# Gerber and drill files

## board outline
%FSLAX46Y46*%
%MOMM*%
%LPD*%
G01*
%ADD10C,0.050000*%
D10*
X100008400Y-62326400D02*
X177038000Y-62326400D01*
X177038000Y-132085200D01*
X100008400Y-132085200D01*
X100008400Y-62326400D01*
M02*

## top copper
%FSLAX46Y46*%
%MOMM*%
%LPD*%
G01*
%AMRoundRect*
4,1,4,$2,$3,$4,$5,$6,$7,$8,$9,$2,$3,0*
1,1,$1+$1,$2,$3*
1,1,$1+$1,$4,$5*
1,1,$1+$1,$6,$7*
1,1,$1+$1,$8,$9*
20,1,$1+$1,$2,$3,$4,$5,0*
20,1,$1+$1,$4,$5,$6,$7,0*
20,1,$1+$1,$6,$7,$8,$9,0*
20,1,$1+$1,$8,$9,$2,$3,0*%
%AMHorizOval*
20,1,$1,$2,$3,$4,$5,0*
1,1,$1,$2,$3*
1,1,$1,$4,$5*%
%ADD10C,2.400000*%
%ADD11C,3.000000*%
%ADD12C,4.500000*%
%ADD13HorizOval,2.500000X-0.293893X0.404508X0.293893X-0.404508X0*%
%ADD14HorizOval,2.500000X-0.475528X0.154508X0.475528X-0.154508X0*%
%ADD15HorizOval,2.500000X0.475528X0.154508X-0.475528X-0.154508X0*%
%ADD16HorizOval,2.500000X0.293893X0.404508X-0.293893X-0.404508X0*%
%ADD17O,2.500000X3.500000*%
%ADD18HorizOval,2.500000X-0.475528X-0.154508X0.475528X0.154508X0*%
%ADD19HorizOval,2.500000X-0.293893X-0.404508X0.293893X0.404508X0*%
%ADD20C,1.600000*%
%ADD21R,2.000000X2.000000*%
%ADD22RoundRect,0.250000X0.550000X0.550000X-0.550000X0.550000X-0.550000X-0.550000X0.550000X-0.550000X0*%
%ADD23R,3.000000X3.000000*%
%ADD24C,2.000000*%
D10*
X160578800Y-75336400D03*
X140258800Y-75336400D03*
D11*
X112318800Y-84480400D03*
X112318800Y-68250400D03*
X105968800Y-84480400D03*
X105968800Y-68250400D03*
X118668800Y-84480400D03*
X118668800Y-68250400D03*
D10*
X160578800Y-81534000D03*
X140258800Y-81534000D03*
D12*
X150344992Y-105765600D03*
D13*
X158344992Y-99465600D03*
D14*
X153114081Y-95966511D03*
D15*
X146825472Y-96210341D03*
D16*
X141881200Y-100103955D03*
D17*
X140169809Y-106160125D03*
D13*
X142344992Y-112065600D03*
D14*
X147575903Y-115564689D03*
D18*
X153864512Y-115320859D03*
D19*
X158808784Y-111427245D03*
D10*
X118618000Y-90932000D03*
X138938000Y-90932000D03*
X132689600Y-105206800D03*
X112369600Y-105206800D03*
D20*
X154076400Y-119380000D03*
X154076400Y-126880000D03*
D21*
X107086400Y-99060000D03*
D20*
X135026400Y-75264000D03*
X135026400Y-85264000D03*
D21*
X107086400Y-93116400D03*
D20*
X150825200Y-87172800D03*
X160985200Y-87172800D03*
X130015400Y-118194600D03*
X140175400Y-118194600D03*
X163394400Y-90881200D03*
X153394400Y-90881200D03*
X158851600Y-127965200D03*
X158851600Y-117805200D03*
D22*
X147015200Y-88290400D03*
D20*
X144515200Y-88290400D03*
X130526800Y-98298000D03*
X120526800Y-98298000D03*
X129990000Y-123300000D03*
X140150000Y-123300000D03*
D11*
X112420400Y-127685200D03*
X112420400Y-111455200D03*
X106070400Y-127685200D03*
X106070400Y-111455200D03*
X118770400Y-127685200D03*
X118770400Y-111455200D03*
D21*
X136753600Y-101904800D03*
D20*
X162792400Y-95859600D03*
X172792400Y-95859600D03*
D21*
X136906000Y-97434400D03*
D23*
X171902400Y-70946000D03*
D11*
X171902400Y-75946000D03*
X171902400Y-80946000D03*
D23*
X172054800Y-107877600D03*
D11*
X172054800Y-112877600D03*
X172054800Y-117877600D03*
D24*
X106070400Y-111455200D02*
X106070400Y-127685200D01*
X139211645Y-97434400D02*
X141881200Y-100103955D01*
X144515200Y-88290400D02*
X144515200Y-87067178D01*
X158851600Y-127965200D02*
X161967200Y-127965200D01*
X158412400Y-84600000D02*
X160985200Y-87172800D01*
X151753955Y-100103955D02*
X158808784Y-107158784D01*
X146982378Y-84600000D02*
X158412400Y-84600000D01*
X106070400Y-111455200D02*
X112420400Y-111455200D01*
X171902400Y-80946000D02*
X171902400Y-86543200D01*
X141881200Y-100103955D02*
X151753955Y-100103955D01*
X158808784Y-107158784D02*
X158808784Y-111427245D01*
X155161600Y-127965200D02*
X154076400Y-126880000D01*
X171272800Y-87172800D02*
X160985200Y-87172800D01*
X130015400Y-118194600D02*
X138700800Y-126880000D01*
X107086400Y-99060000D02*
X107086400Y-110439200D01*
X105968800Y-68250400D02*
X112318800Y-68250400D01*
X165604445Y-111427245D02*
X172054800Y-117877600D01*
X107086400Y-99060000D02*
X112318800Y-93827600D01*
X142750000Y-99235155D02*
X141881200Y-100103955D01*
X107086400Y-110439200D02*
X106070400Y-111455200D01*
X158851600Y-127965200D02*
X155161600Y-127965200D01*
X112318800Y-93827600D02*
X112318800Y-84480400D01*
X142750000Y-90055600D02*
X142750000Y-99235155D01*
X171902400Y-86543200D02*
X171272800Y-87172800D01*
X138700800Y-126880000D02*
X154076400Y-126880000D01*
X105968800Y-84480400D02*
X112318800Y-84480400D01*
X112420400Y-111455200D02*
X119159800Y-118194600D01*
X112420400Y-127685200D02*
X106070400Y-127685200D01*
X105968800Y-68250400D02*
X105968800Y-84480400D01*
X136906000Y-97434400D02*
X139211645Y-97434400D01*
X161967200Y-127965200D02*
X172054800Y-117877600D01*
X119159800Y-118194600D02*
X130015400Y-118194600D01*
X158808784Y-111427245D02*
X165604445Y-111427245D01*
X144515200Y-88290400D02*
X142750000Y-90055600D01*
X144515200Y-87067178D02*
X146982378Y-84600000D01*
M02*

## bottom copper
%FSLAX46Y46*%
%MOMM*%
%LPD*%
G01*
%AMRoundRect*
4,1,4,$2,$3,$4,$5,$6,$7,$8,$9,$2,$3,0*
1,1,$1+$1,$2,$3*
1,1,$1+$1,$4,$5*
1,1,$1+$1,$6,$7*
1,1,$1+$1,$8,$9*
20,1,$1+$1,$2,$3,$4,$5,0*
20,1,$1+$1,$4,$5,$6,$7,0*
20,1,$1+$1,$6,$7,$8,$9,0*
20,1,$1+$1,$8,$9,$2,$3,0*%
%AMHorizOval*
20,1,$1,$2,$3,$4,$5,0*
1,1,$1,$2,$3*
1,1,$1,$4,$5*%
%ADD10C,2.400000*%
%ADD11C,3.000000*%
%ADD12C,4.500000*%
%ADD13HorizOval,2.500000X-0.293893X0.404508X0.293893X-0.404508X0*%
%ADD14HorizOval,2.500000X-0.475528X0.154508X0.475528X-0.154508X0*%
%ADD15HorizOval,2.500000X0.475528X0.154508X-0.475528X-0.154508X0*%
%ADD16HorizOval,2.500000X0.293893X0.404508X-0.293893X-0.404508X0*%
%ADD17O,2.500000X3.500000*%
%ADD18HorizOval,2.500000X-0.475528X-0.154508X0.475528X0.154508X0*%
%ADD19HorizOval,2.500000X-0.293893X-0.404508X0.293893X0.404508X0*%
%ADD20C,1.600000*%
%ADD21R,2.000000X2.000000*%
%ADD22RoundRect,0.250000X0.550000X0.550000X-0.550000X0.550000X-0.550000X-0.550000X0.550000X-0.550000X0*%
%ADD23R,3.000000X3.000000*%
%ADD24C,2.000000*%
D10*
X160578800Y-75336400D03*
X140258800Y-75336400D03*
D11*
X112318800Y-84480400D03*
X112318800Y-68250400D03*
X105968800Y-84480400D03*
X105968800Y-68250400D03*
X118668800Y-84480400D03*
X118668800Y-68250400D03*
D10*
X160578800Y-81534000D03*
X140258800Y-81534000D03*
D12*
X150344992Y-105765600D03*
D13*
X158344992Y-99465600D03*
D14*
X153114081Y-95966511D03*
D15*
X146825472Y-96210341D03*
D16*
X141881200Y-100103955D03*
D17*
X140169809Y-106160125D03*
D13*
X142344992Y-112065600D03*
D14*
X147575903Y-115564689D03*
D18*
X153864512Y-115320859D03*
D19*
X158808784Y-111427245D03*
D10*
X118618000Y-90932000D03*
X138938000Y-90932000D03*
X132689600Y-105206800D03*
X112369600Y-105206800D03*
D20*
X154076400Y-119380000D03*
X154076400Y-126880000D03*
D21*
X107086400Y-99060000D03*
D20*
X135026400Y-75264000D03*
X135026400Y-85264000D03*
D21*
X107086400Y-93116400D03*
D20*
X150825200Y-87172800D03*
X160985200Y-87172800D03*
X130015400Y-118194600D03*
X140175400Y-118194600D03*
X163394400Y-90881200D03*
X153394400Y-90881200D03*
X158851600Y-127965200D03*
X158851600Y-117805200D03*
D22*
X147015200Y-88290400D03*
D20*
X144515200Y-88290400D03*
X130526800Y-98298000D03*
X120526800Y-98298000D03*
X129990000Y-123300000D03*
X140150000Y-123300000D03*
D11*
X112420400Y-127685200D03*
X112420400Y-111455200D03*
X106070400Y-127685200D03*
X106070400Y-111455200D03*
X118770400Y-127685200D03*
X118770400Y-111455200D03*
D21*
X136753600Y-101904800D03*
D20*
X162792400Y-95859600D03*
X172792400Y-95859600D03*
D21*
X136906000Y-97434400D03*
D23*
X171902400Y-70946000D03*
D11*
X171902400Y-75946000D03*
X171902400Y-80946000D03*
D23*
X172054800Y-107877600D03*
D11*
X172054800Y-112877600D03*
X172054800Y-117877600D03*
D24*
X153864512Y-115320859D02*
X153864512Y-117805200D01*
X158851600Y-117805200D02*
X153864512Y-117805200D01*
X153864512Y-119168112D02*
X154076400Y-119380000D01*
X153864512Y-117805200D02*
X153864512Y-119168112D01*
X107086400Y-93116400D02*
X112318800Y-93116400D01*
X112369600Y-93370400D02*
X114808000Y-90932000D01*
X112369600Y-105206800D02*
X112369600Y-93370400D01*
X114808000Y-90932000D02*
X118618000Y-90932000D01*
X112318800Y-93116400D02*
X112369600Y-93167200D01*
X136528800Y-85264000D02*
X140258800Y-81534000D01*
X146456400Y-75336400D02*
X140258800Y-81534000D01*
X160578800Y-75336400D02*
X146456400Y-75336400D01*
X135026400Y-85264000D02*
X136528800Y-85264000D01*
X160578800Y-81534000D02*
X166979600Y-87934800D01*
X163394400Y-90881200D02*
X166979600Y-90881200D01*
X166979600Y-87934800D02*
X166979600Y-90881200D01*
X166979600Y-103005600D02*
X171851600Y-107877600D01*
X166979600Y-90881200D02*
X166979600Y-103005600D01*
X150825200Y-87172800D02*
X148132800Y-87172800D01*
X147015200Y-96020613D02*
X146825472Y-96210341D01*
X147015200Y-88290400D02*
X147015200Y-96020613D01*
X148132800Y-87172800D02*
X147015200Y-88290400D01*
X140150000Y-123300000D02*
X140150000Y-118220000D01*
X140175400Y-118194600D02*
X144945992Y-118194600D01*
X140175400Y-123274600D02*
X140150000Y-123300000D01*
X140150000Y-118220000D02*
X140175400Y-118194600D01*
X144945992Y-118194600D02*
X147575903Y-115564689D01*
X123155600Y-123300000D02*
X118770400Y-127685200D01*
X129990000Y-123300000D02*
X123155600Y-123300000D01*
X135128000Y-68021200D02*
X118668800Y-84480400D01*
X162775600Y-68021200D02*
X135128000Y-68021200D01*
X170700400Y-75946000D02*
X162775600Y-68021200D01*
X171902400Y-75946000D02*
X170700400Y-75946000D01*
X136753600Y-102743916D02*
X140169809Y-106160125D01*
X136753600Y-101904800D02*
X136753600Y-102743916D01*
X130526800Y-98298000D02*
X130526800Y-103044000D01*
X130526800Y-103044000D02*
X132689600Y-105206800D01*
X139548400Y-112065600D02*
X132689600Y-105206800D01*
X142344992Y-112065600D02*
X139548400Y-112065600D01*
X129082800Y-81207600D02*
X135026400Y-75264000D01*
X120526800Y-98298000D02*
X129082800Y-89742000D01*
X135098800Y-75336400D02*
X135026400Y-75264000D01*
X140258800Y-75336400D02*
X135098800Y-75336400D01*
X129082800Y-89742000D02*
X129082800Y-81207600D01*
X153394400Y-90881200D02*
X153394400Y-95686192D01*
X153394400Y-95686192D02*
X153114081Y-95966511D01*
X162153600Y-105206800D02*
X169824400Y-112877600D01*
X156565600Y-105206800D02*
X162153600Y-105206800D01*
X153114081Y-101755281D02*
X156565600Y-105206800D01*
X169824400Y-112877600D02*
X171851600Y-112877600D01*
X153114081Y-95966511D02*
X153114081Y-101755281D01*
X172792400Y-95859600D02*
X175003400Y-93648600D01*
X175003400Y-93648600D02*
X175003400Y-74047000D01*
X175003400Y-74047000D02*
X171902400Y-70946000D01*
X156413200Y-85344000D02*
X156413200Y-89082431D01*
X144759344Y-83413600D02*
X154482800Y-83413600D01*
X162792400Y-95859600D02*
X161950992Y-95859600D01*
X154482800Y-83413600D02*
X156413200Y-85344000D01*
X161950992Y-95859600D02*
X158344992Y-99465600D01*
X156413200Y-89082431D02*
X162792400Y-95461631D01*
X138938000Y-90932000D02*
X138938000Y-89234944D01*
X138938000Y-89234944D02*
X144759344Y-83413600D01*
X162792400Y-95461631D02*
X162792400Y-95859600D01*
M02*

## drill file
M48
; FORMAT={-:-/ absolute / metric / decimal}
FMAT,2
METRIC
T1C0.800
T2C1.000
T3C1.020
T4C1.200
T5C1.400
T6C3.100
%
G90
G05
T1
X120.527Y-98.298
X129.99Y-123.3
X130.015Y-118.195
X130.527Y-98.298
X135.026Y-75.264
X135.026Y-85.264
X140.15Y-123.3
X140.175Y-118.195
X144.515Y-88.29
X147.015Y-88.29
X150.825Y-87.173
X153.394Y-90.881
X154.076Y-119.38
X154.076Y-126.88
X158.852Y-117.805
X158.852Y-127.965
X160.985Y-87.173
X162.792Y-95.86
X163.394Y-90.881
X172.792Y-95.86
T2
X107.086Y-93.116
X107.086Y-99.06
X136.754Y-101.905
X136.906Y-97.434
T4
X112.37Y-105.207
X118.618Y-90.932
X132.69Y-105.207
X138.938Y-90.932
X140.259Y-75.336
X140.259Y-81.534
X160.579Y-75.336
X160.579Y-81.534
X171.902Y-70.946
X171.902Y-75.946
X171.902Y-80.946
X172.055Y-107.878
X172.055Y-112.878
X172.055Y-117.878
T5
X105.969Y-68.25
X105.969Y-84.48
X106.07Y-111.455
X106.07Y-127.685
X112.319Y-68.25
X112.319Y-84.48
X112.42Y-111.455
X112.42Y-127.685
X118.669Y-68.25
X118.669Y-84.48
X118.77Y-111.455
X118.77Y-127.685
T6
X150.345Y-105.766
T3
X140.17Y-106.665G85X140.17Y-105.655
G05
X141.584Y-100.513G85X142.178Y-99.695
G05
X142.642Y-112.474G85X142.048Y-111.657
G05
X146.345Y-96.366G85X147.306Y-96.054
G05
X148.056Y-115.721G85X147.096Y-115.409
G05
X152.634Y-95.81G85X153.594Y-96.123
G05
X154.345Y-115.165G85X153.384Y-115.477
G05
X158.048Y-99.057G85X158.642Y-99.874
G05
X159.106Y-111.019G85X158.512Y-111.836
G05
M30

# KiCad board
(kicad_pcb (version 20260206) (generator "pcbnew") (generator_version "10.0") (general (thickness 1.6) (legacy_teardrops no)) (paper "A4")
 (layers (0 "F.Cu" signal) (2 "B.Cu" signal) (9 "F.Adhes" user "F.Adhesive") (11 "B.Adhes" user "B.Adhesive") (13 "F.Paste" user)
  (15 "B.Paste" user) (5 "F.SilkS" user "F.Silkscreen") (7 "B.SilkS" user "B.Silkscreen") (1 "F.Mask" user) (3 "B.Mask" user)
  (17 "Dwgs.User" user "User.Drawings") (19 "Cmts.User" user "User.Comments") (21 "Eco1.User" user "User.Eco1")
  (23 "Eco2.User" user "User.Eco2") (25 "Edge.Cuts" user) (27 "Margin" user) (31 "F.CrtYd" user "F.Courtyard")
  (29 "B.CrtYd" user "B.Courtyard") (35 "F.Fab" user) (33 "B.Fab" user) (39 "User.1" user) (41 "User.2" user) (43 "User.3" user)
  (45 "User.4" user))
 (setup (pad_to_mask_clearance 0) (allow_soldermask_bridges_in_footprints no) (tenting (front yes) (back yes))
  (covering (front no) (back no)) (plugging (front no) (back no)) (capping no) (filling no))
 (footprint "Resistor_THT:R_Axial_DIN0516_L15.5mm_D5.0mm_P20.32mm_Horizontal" (layer "F.Cu") (at 160.5788 75.3364 180)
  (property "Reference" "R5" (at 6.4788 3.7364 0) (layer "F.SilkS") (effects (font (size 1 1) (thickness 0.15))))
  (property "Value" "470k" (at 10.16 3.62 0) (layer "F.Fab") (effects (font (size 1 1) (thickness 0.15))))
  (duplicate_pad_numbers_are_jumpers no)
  (pad "1" thru_hole circle (at 0 0 180) (size 2.4 2.4) (drill 1.2) (layers "*.Cu" "*.Mask") (remove_unused_layers no) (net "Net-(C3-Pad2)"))
  (pad "2" thru_hole circle (at 20.32 0 180) (size 2.4 2.4) (drill 1.2) (layers "*.Cu" "*.Mask") (remove_unused_layers no)
   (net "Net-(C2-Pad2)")))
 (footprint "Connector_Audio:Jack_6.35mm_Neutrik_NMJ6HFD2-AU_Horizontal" (layer "F.Cu") (at 118.6688 84.4804 180)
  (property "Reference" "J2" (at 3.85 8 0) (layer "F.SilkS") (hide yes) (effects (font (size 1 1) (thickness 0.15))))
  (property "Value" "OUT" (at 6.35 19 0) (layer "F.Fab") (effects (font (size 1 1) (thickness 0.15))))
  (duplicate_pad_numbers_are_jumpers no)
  (pad "R" thru_hole circle (at 6.35 0 180) (size 3 3) (drill 1.4) (layers "*.Cu" "*.Mask") (remove_unused_layers no) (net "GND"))
  (pad "RN" thru_hole circle (at 6.35 16.23 180) (size 3 3) (drill 1.4) (layers "*.Cu" "*.Mask") (remove_unused_layers no) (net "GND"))
  (pad "S" thru_hole circle (at 12.7 0 180) (size 3 3) (drill 1.4) (layers "*.Cu" "*.Mask") (remove_unused_layers no) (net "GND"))
  (pad "SN" thru_hole circle (at 12.7 16.23 180) (size 3 3) (drill 1.4) (layers "*.Cu" "*.Mask") (remove_unused_layers no) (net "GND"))
  (pad "T" thru_hole circle (at 0 0 180) (size 3 3) (drill 1.4) (layers "*.Cu" "*.Mask") (remove_unused_layers no) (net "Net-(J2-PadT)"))
  (pad "TN" thru_hole circle (at 0 16.23 180) (size 3 3) (drill 1.4) (layers "*.Cu" "*.Mask") (remove_unused_layers no)
   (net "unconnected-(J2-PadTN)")))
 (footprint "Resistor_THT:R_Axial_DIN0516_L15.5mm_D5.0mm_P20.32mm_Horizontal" (layer "F.Cu") (at 160.5788 81.534 180)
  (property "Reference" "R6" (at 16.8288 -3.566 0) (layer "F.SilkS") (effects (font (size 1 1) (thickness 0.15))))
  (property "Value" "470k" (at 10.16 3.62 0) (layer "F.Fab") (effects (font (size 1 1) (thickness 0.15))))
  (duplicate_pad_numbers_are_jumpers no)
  (pad "1" thru_hole circle (at 0 0 180) (size 2.4 2.4) (drill 1.2) (layers "*.Cu" "*.Mask") (remove_unused_layers no) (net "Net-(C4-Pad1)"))
  (pad "2" thru_hole circle (at 20.32 0 180) (size 2.4 2.4) (drill 1.2) (layers "*.Cu" "*.Mask") (remove_unused_layers no)
   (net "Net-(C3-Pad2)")))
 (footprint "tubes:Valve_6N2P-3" (layer "F.Cu") (at 158.344992 99.4656 90)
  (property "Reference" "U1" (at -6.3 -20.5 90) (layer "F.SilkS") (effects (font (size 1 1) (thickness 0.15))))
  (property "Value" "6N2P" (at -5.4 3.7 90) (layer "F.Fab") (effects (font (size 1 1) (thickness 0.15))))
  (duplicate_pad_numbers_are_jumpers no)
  (pad "" np_thru_hole circle (at -6.3 -8 90) (size 4.5 4.5) (drill 3.1) (layers "*.Cu" "*.Mask"))
  (pad "1" thru_hole oval (at 0 0 36) (size 2.5 3.5) (drill oval 1.02 2.03) (layers "*.Cu" "*.Mask") (remove_unused_layers no)
   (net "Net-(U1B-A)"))
  (pad "2" thru_hole oval (at 3.499089 -5.230911 72) (size 2.5 3.5) (drill oval 1.02 2.03) (layers "*.Cu" "*.Mask")
   (remove_unused_layers no) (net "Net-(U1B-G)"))
  (pad "3" thru_hole oval (at 3.255259 -11.51952 108) (size 2.5 3.5) (drill oval 1.02 2.03) (layers "*.Cu" "*.Mask")
   (remove_unused_layers no) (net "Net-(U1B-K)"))
  (pad "4" thru_hole oval (at -0.638355 -16.463792 144) (size 2.5 3.5) (drill oval 1.02 2.03) (layers "*.Cu" "*.Mask")
   (remove_unused_layers no) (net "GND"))
  (pad "5" thru_hole oval (at -6.694525 -18.175183 180) (size 2.5 3.5) (drill oval 1.02 2.03) (layers "*.Cu" "*.Mask")
   (remove_unused_layers no) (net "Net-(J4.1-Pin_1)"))
  (pad "6" thru_hole oval (at -12.6 -16 216) (size 2.5 3.5) (drill oval 1.02 2.03) (layers "*.Cu" "*.Mask") (remove_unused_layers no)
   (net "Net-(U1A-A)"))
  (pad "7" thru_hole oval (at -16.099089 -10.769089 252) (size 2.5 3.5) (drill oval 1.02 2.03) (layers "*.Cu" "*.Mask")
   (remove_unused_layers no) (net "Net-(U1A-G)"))
  (pad "8" thru_hole oval (at -15.855259 -4.48048 288) (size 2.5 3.5) (drill oval 1.02 2.03) (layers "*.Cu" "*.Mask")
   (remove_unused_layers no) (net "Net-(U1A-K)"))
  (pad "9" thru_hole oval (at -11.961645 0.463792 324) (size 2.5 3.5) (drill oval 1.02 2.03) (layers "*.Cu" "*.Mask")
   (remove_unused_layers no) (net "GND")))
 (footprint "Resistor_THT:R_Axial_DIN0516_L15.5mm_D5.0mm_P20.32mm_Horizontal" (layer "F.Cu") (at 118.618 90.932)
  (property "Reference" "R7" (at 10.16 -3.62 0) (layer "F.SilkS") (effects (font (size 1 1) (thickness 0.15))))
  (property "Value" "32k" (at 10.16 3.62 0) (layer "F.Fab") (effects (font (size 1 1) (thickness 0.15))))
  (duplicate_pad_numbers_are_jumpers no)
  (pad "1" thru_hole circle (at 0 0) (size 2.4 2.4) (drill 1.2) (layers "*.Cu" "*.Mask") (remove_unused_layers no) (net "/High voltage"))
  (pad "2" thru_hole circle (at 20.32 0) (size 2.4 2.4) (drill 1.2) (layers "*.Cu" "*.Mask") (remove_unused_layers no) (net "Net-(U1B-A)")))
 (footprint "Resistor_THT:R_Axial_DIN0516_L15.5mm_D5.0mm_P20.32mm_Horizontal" (layer "F.Cu") (at 132.6896 105.2068 180)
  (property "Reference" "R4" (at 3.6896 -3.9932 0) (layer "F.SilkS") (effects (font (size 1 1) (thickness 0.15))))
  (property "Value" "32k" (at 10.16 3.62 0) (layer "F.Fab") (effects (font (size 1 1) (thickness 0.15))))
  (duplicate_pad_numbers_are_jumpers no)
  (pad "1" thru_hole circle (at 0 0 180) (size 2.4 2.4) (drill 1.2) (layers "*.Cu" "*.Mask") (remove_unused_layers no) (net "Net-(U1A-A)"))
  (pad "2" thru_hole circle (at 20.32 0 180) (size 2.4 2.4) (drill 1.2) (layers "*.Cu" "*.Mask") (remove_unused_layers no)
   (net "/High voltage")))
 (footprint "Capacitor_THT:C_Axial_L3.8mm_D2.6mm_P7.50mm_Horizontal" (layer "F.Cu") (at 154.0764 119.38 -90)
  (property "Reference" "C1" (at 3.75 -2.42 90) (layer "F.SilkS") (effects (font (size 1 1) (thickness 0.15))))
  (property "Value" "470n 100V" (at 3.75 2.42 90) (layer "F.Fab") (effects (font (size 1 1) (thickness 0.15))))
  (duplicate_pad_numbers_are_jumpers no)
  (pad "1" thru_hole circle (at 0 0 270) (size 1.6 1.6) (drill 0.8) (layers "*.Cu" "*.Mask") (remove_unused_layers no) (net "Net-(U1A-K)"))
  (pad "2" thru_hole circle (at 7.5 0 270) (size 1.6 1.6) (drill 0.8) (layers "*.Cu" "*.Mask") (remove_unused_layers no) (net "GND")))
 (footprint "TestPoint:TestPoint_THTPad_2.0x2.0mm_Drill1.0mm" (layer "F.Cu") (at 107.0864 99.06)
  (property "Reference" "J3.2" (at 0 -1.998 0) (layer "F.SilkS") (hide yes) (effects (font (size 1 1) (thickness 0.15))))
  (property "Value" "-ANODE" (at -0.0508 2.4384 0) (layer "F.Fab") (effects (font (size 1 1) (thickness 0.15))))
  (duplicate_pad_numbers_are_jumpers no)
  (pad "1" thru_hole rect (at 0 0) (size 2 2) (drill 1) (layers "*.Cu" "*.Mask") (remove_unused_layers no) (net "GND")))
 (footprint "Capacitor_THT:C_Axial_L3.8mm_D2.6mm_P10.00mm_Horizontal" (layer "F.Cu") (at 135.0264 75.264 -90)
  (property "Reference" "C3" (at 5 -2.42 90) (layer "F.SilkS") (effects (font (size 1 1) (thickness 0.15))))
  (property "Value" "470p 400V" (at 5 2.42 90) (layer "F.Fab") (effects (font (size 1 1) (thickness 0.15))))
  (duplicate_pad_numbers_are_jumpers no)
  (pad "1" thru_hole circle (at 0 0 270) (size 1.6 1.6) (drill 0.8) (layers "*.Cu" "*.Mask") (remove_unused_layers no) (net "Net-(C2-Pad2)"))
  (pad "2" thru_hole circle (at 10 0 270) (size 1.6 1.6) (drill 0.8) (layers "*.Cu" "*.Mask") (remove_unused_layers no)
   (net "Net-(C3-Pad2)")))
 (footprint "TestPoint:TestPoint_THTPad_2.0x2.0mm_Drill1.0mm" (layer "F.Cu") (at 107.0864 93.1164 180)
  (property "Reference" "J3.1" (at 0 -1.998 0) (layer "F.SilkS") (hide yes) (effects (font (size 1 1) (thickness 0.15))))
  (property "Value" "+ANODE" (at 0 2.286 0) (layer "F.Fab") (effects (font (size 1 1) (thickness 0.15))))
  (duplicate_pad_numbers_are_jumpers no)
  (pad "1" thru_hole rect (at 0 0 180) (size 2 2) (drill 1) (layers "*.Cu" "*.Mask") (remove_unused_layers no) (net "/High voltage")))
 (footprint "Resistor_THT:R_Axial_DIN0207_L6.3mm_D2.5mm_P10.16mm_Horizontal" (layer "F.Cu") (at 150.8252 87.1728)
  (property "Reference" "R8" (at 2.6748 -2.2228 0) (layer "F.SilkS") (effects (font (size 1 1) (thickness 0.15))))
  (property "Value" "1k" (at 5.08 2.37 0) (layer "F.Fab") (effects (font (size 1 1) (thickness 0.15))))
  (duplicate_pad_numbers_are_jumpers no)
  (pad "1" thru_hole circle (at 0 0) (size 1.6 1.6) (drill 0.8) (layers "*.Cu" "*.Mask") (remove_unused_layers no) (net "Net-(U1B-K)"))
  (pad "2" thru_hole circle (at 10.16 0) (size 1.6 1.6) (drill 0.8) (layers "*.Cu" "*.Mask") (remove_unused_layers no) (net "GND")))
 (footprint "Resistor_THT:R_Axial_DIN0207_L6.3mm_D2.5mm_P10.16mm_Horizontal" (layer "F.Cu") (at 130.0154 118.1946)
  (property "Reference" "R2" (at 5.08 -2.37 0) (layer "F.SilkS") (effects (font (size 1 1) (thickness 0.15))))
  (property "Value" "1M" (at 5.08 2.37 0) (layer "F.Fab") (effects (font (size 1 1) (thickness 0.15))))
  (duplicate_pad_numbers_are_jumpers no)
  (pad "1" thru_hole circle (at 0 0) (size 1.6 1.6) (drill 0.8) (layers "*.Cu" "*.Mask") (remove_unused_layers no) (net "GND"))
  (pad "2" thru_hole circle (at 10.16 0) (size 1.6 1.6) (drill 0.8) (layers "*.Cu" "*.Mask") (remove_unused_layers no) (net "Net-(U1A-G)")))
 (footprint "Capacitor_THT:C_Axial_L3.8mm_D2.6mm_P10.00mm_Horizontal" (layer "F.Cu") (at 163.3944 90.8812 180)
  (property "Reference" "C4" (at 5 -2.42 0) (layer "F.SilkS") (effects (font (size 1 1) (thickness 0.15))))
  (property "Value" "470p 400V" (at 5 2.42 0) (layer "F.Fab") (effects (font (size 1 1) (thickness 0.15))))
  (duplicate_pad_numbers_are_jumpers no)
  (pad "1" thru_hole circle (at 0 0 180) (size 1.6 1.6) (drill 0.8) (layers "*.Cu" "*.Mask") (remove_unused_layers no) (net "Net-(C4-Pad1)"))
  (pad "2" thru_hole circle (at 10 0 180) (size 1.6 1.6) (drill 0.8) (layers "*.Cu" "*.Mask") (remove_unused_layers no) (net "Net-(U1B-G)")))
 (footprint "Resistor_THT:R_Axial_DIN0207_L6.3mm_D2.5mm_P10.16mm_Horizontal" (layer "F.Cu") (at 158.8516 127.9652 90)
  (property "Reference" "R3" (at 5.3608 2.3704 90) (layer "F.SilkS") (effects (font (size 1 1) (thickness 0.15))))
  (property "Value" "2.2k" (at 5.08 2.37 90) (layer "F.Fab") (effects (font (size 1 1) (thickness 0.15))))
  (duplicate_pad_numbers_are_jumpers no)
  (pad "1" thru_hole circle (at 0 0 90) (size 1.6 1.6) (drill 0.8) (layers "*.Cu" "*.Mask") (remove_unused_layers no) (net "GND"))
  (pad "2" thru_hole circle (at 10.16 0 90) (size 1.6 1.6) (drill 0.8) (layers "*.Cu" "*.Mask") (remove_unused_layers no)
   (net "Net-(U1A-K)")))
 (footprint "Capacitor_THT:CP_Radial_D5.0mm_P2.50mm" (layer "F.Cu") (at 147.0152 88.2904 180)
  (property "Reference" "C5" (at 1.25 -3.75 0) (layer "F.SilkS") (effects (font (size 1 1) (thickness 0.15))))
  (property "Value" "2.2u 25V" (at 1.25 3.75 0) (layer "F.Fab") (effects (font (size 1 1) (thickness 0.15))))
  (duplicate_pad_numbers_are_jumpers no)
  (pad "1" thru_hole roundrect (at 0 0 180) (size 1.6 1.6) (drill 0.8) (layers "*.Cu" "*.Mask") (remove_unused_layers no)
   (roundrect_rratio 0.15625) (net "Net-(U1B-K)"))
  (pad "2" thru_hole circle (at 2.5 0 180) (size 1.6 1.6) (drill 0.8) (layers "*.Cu" "*.Mask") (remove_unused_layers no) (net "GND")))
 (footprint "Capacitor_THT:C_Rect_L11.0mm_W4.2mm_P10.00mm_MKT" (layer "F.Cu") (at 130.5268 98.298 180)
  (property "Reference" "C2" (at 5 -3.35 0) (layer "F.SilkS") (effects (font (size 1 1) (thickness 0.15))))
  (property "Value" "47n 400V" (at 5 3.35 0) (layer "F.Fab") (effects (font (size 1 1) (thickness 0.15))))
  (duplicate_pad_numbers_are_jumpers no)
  (pad "1" thru_hole circle (at 0 0 180) (size 1.6 1.6) (drill 0.8) (layers "*.Cu" "*.Mask") (remove_unused_layers no) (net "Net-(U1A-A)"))
  (pad "2" thru_hole circle (at 10 0 180) (size 1.6 1.6) (drill 0.8) (layers "*.Cu" "*.Mask") (remove_unused_layers no)
   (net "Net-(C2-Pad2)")))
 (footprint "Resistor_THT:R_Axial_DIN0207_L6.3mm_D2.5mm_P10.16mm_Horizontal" (layer "F.Cu") (at 129.99 123.3)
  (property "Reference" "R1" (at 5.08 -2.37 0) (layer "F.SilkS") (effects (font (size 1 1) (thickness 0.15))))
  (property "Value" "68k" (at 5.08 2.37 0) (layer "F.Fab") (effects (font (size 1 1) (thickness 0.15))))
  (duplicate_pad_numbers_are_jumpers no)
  (pad "1" thru_hole circle (at 0 0) (size 1.6 1.6) (drill 0.8) (layers "*.Cu" "*.Mask") (remove_unused_layers no) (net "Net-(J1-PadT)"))
  (pad "2" thru_hole circle (at 10.16 0) (size 1.6 1.6) (drill 0.8) (layers "*.Cu" "*.Mask") (remove_unused_layers no) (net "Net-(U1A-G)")))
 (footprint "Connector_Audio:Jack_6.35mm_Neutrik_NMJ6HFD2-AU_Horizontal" (layer "F.Cu") (at 118.7704 127.6852 180)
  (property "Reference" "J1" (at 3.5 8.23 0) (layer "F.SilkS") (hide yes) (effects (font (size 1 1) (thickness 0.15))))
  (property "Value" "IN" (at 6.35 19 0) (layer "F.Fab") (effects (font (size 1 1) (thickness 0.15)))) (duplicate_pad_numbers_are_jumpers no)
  (pad "R" thru_hole circle (at 6.35 0 180) (size 3 3) (drill 1.4) (layers "*.Cu" "*.Mask") (remove_unused_layers no) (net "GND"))
  (pad "RN" thru_hole circle (at 6.35 16.23 180) (size 3 3) (drill 1.4) (layers "*.Cu" "*.Mask") (remove_unused_layers no) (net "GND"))
  (pad "S" thru_hole circle (at 12.7 0 180) (size 3 3) (drill 1.4) (layers "*.Cu" "*.Mask") (remove_unused_layers no) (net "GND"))
  (pad "SN" thru_hole circle (at 12.7 16.23 180) (size 3 3) (drill 1.4) (layers "*.Cu" "*.Mask") (remove_unused_layers no) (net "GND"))
  (pad "T" thru_hole circle (at 0 0 180) (size 3 3) (drill 1.4) (layers "*.Cu" "*.Mask") (remove_unused_layers no) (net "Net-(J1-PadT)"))
  (pad "TN" thru_hole circle (at 0 16.23 180) (size 3 3) (drill 1.4) (layers "*.Cu" "*.Mask") (remove_unused_layers no)
   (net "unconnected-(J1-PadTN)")))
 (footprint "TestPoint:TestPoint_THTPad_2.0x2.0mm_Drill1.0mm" (layer "F.Cu") (at 136.7536 101.9048 -90)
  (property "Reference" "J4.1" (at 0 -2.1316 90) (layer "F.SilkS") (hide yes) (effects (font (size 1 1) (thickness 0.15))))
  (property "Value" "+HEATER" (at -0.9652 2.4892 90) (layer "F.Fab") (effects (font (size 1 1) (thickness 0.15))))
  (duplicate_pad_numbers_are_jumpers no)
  (pad "1" thru_hole rect (at 0 0 270) (size 2 2) (drill 1) (layers "*.Cu" "*.Mask") (remove_unused_layers no) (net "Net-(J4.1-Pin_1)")))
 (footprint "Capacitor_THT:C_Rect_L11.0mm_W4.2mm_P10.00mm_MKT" (layer "F.Cu") (at 162.7924 95.8596)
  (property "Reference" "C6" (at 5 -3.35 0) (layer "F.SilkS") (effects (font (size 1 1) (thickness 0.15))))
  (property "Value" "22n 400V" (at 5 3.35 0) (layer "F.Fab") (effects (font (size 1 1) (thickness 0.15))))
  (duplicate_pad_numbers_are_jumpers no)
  (pad "1" thru_hole circle (at 0 0) (size 1.6 1.6) (drill 0.8) (layers "*.Cu" "*.Mask") (remove_unused_layers no) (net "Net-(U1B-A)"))
  (pad "2" thru_hole circle (at 10 0) (size 1.6 1.6) (drill 0.8) (layers "*.Cu" "*.Mask") (remove_unused_layers no) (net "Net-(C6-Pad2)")))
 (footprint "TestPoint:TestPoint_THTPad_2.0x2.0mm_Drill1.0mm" (layer "F.Cu") (at 136.906 97.4344 -90)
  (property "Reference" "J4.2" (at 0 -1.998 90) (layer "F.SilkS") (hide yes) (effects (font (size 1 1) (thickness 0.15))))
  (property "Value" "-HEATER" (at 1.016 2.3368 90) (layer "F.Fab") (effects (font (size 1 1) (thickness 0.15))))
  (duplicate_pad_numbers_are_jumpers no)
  (pad "1" thru_hole rect (at 0 0 270) (size 2 2) (drill 1) (layers "*.Cu" "*.Mask") (remove_unused_layers no) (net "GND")))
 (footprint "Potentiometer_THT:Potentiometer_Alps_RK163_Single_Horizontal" (layer "B.Cu") (at 171.9024 70.946 180)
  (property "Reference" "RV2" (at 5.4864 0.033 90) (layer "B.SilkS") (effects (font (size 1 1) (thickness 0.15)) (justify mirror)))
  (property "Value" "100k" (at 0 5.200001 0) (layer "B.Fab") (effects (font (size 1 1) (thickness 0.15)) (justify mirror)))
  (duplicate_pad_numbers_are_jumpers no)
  (pad "1" thru_hole rect (at 0 0) (size 3 3) (drill 1.2) (layers "*.Cu" "*.Mask") (remove_unused_layers no) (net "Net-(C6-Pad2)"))
  (pad "2" thru_hole circle (at 0 -5) (size 3 3) (drill 1.2) (layers "*.Cu" "*.Mask") (remove_unused_layers no) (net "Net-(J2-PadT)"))
  (pad "3" thru_hole circle (at 0 -10) (size 3 3) (drill 1.2) (layers "*.Cu" "*.Mask") (remove_unused_layers no) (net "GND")))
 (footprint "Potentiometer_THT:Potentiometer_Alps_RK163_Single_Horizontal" (layer "B.Cu") (at 172.0548 107.8776 180)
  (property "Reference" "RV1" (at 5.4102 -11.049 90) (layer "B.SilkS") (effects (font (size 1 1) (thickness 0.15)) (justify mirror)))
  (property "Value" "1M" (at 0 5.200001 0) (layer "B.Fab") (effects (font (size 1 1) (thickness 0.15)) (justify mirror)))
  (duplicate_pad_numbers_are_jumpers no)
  (pad "1" thru_hole rect (at 0 0) (size 3 3) (drill 1.2) (layers "*.Cu" "*.Mask") (remove_unused_layers no) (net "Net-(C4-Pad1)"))
  (pad "2" thru_hole circle (at 0 -5) (size 3 3) (drill 1.2) (layers "*.Cu" "*.Mask") (remove_unused_layers no) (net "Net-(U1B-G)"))
  (pad "3" thru_hole circle (at 0 -10) (size 3 3) (drill 1.2) (layers "*.Cu" "*.Mask") (remove_unused_layers no) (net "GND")))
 (gr_rect (start 100.0084 62.3264) (end 177.038 132.0852) (stroke (width 0.05) (type default)) (fill no) (layer "Edge.Cuts"))
 (segment (start 106.0704 111.4552) (end 106.0704 127.6852) (width 2) (layer "F.Cu") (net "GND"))
 (segment (start 139.211645 97.4344) (end 141.8812 100.103955) (width 2) (layer "F.Cu") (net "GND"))
 (segment (start 144.5152 88.2904) (end 144.5152 87.067178) (width 2) (layer "F.Cu") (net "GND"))
 (segment (start 158.8516 127.9652) (end 161.9672 127.9652) (width 2) (layer "F.Cu") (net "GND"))
 (segment (start 158.4124 84.6) (end 160.9852 87.1728) (width 2) (layer "F.Cu") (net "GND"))
 (segment (start 151.753955 100.103955) (end 158.808784 107.158784) (width 2) (layer "F.Cu") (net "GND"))
 (segment (start 146.982378 84.6) (end 158.4124 84.6) (width 2) (layer "F.Cu") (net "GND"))
 (segment (start 106.0704 111.4552) (end 112.4204 111.4552) (width 2) (layer "F.Cu") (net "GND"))
 (segment (start 171.9024 80.946) (end 171.9024 86.5432) (width 2) (layer "F.Cu") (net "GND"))
 (segment (start 141.8812 100.103955) (end 151.753955 100.103955) (width 2) (layer "F.Cu") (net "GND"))
 (segment (start 158.808784 107.158784) (end 158.808784 111.427245) (width 2) (layer "F.Cu") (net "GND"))
 (segment (start 155.1616 127.9652) (end 154.0764 126.88) (width 2) (layer "F.Cu") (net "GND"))
 (segment (start 171.2728 87.1728) (end 160.9852 87.1728) (width 2) (layer "F.Cu") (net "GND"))
 (segment (start 130.0154 118.1946) (end 138.7008 126.88) (width 2) (layer "F.Cu") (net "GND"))
 (segment (start 107.0864 99.06) (end 107.0864 110.4392) (width 2) (layer "F.Cu") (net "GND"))
 (segment (start 105.9688 68.2504) (end 112.3188 68.2504) (width 2) (layer "F.Cu") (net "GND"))
 (segment (start 165.604445 111.427245) (end 172.0548 117.8776) (width 2) (layer "F.Cu") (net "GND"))
 (segment (start 107.0864 99.06) (end 112.3188 93.8276) (width 2) (layer "F.Cu") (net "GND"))
 (segment (start 142.75 99.235155) (end 141.8812 100.103955) (width 2) (layer "F.Cu") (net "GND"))
 (segment (start 107.0864 110.4392) (end 106.0704 111.4552) (width 2) (layer "F.Cu") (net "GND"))
 (segment (start 158.8516 127.9652) (end 155.1616 127.9652) (width 2) (layer "F.Cu") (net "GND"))
 (segment (start 112.3188 93.8276) (end 112.3188 84.4804) (width 2) (layer "F.Cu") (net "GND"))
 (segment (start 142.75 90.0556) (end 142.75 99.235155) (width 2) (layer "F.Cu") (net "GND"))
 (segment (start 171.9024 86.5432) (end 171.2728 87.1728) (width 2) (layer "F.Cu") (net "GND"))
 (segment (start 138.7008 126.88) (end 154.0764 126.88) (width 2) (layer "F.Cu") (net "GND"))
 (segment (start 105.9688 84.4804) (end 112.3188 84.4804) (width 2) (layer "F.Cu") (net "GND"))
 (segment (start 112.4204 111.4552) (end 119.1598 118.1946) (width 2) (layer "F.Cu") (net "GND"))
 (segment (start 112.4204 127.6852) (end 106.0704 127.6852) (width 2) (layer "F.Cu") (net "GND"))
 (segment (start 105.9688 68.2504) (end 105.9688 84.4804) (width 2) (layer "F.Cu") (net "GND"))
 (segment (start 136.906 97.4344) (end 139.211645 97.4344) (width 2) (layer "F.Cu") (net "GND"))
 (segment (start 161.9672 127.9652) (end 172.0548 117.8776) (width 2) (layer "F.Cu") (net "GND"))
 (segment (start 119.1598 118.1946) (end 130.0154 118.1946) (width 2) (layer "F.Cu") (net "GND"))
 (segment (start 158.808784 111.427245) (end 165.604445 111.427245) (width 2) (layer "F.Cu") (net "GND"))
 (segment (start 144.5152 88.2904) (end 142.75 90.0556) (width 2) (layer "F.Cu") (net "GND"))
 (segment (start 144.5152 87.067178) (end 146.982378 84.6) (width 2) (layer "F.Cu") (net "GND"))
 (segment (start 153.864512 115.320859) (end 153.864512 117.8052) (width 2) (layer "B.Cu") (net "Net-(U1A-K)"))
 (segment (start 158.8516 117.8052) (end 153.864512 117.8052) (width 2) (layer "B.Cu") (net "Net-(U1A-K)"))
 (segment (start 153.864512 119.168112) (end 154.0764 119.38) (width 2) (layer "B.Cu") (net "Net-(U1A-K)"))
 (segment (start 153.864512 117.8052) (end 153.864512 119.168112) (width 2) (layer "B.Cu") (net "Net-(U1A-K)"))
 (segment (start 107.0864 93.1164) (end 112.3188 93.1164) (width 2) (layer "B.Cu") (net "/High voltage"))
 (segment (start 112.3696 93.3704) (end 114.808 90.932) (width 2) (layer "B.Cu") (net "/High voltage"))
 (segment (start 112.3696 105.2068) (end 112.3696 93.3704) (width 2) (layer "B.Cu") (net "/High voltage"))
 (segment (start 114.808 90.932) (end 118.618 90.932) (width 2) (layer "B.Cu") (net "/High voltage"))
 (segment (start 112.3188 93.1164) (end 112.3696 93.1672) (width 2) (layer "B.Cu") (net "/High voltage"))
 (segment (start 136.5288 85.264) (end 140.2588 81.534) (width 2) (layer "B.Cu") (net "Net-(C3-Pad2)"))
 (segment (start 146.4564 75.3364) (end 140.2588 81.534) (width 2) (layer "B.Cu") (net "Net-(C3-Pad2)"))
 (segment (start 160.5788 75.3364) (end 146.4564 75.3364) (width 2) (layer "B.Cu") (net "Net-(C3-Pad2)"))
 (segment (start 135.0264 85.264) (end 136.5288 85.264) (width 2) (layer "B.Cu") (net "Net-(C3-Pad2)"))
 (segment (start 160.5788 81.534) (end 166.9796 87.9348) (width 2) (layer "B.Cu") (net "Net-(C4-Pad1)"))
 (segment (start 163.3944 90.8812) (end 166.9796 90.8812) (width 2) (layer "B.Cu") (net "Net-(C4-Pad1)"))
 (segment (start 166.9796 87.9348) (end 166.9796 90.8812) (width 2) (layer "B.Cu") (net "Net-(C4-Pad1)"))
 (segment (start 166.9796 103.0056) (end 171.8516 107.8776) (width 2) (layer "B.Cu") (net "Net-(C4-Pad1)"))
 (segment (start 166.9796 90.8812) (end 166.9796 103.0056) (width 2) (layer "B.Cu") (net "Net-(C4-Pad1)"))
 (segment (start 150.8252 87.1728) (end 148.1328 87.1728) (width 2) (layer "B.Cu") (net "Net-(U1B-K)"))
 (segment (start 147.0152 96.020613) (end 146.825472 96.210341) (width 2) (layer "B.Cu") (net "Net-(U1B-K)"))
 (segment (start 147.0152 88.2904) (end 147.0152 96.020613) (width 2) (layer "B.Cu") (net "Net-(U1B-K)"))
 (segment (start 148.1328 87.1728) (end 147.0152 88.2904) (width 2) (layer "B.Cu") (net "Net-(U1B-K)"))
 (segment (start 140.15 123.3) (end 140.15 118.22) (width 2) (layer "B.Cu") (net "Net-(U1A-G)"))
 (segment (start 140.1754 118.1946) (end 144.945992 118.1946) (width 2) (layer "B.Cu") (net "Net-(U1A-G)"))
 (segment (start 140.1754 123.2746) (end 140.15 123.3) (width 2) (layer "B.Cu") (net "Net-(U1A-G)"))
 (segment (start 140.15 118.22) (end 140.1754 118.1946) (width 2) (layer "B.Cu") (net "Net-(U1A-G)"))
 (segment (start 144.945992 118.1946) (end 147.575903 115.564689) (width 2) (layer "B.Cu") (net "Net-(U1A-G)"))
 (segment (start 123.1556 123.3) (end 118.7704 127.6852) (width 2) (layer "B.Cu") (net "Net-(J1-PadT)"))
 (segment (start 129.99 123.3) (end 123.1556 123.3) (width 2) (layer "B.Cu") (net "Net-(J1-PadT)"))
 (segment (start 135.128 68.0212) (end 118.6688 84.4804) (width 2) (layer "B.Cu") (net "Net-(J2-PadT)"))
 (segment (start 162.7756 68.0212) (end 135.128 68.0212) (width 2) (layer "B.Cu") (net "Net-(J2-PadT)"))
 (segment (start 170.7004 75.946) (end 162.7756 68.0212) (width 2) (layer "B.Cu") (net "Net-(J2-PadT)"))
 (segment (start 171.9024 75.946) (end 170.7004 75.946) (width 2) (layer "B.Cu") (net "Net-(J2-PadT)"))
 (segment (start 136.7536 102.743916) (end 140.169809 106.160125) (width 2) (layer "B.Cu") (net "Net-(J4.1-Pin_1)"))
 (segment (start 136.7536 101.9048) (end 136.7536 102.743916) (width 2) (layer "B.Cu") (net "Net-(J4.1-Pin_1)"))
 (segment (start 130.5268 98.298) (end 130.5268 103.044) (width 2) (layer "B.Cu") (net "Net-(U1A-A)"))
 (segment (start 130.5268 103.044) (end 132.6896 105.2068) (width 2) (layer "B.Cu") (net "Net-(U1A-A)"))
 (segment (start 139.5484 112.0656) (end 132.6896 105.2068) (width 2) (layer "B.Cu") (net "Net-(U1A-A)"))
 (segment (start 142.344992 112.0656) (end 139.5484 112.0656) (width 2) (layer "B.Cu") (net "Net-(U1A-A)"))
 (segment (start 129.0828 81.2076) (end 135.0264 75.264) (width 2) (layer "B.Cu") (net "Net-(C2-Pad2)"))
 (segment (start 120.5268 98.298) (end 129.0828 89.742) (width 2) (layer "B.Cu") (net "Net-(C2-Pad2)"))
 (segment (start 135.0988 75.3364) (end 135.0264 75.264) (width 2) (layer "B.Cu") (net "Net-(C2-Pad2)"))
 (segment (start 140.2588 75.3364) (end 135.0988 75.3364) (width 2) (layer "B.Cu") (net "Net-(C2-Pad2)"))
 (segment (start 129.0828 89.742) (end 129.0828 81.2076) (width 2) (layer "B.Cu") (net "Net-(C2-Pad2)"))
 (segment (start 153.3944 90.8812) (end 153.3944 95.686192) (width 2) (layer "B.Cu") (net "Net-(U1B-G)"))
 (segment (start 153.3944 95.686192) (end 153.114081 95.966511) (width 2) (layer "B.Cu") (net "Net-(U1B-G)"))
 (segment (start 162.1536 105.2068) (end 169.8244 112.8776) (width 2) (layer "B.Cu") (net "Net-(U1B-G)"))
 (segment (start 156.5656 105.2068) (end 162.1536 105.2068) (width 2) (layer "B.Cu") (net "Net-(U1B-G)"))
 (segment (start 153.114081 101.755281) (end 156.5656 105.2068) (width 2) (layer "B.Cu") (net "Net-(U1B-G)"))
 (segment (start 169.8244 112.8776) (end 171.8516 112.8776) (width 2) (layer "B.Cu") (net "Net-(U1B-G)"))
 (segment (start 153.114081 95.966511) (end 153.114081 101.755281) (width 2) (layer "B.Cu") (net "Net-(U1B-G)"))
 (segment (start 172.7924 95.8596) (end 175.0034 93.6486) (width 2) (layer "B.Cu") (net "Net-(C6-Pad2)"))
 (segment (start 175.0034 93.6486) (end 175.0034 74.047) (width 2) (layer "B.Cu") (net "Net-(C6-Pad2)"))
 (segment (start 175.0034 74.047) (end 171.9024 70.946) (width 2) (layer "B.Cu") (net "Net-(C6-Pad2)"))
 (segment (start 156.4132 85.344) (end 156.4132 89.082431) (width 2) (layer "B.Cu") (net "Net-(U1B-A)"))
 (segment (start 144.759344 83.4136) (end 154.4828 83.4136) (width 2) (layer "B.Cu") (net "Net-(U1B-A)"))
 (segment (start 162.7924 95.8596) (end 161.950992 95.8596) (width 2) (layer "B.Cu") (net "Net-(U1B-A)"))
 (segment (start 154.4828 83.4136) (end 156.4132 85.344) (width 2) (layer "B.Cu") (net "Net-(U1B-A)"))
 (segment (start 161.950992 95.8596) (end 158.344992 99.4656) (width 2) (layer "B.Cu") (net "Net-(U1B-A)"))
 (segment (start 156.4132 89.082431) (end 162.7924 95.461631) (width 2) (layer "B.Cu") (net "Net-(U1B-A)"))
 (segment (start 138.938 90.932) (end 138.938 89.234944) (width 2) (layer "B.Cu") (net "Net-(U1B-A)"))
 (segment (start 138.938 89.234944) (end 144.759344 83.4136) (width 2) (layer "B.Cu") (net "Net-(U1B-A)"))
 (segment (start 162.7924 95.461631) (end 162.7924 95.8596) (width 2) (layer "B.Cu") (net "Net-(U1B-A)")))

